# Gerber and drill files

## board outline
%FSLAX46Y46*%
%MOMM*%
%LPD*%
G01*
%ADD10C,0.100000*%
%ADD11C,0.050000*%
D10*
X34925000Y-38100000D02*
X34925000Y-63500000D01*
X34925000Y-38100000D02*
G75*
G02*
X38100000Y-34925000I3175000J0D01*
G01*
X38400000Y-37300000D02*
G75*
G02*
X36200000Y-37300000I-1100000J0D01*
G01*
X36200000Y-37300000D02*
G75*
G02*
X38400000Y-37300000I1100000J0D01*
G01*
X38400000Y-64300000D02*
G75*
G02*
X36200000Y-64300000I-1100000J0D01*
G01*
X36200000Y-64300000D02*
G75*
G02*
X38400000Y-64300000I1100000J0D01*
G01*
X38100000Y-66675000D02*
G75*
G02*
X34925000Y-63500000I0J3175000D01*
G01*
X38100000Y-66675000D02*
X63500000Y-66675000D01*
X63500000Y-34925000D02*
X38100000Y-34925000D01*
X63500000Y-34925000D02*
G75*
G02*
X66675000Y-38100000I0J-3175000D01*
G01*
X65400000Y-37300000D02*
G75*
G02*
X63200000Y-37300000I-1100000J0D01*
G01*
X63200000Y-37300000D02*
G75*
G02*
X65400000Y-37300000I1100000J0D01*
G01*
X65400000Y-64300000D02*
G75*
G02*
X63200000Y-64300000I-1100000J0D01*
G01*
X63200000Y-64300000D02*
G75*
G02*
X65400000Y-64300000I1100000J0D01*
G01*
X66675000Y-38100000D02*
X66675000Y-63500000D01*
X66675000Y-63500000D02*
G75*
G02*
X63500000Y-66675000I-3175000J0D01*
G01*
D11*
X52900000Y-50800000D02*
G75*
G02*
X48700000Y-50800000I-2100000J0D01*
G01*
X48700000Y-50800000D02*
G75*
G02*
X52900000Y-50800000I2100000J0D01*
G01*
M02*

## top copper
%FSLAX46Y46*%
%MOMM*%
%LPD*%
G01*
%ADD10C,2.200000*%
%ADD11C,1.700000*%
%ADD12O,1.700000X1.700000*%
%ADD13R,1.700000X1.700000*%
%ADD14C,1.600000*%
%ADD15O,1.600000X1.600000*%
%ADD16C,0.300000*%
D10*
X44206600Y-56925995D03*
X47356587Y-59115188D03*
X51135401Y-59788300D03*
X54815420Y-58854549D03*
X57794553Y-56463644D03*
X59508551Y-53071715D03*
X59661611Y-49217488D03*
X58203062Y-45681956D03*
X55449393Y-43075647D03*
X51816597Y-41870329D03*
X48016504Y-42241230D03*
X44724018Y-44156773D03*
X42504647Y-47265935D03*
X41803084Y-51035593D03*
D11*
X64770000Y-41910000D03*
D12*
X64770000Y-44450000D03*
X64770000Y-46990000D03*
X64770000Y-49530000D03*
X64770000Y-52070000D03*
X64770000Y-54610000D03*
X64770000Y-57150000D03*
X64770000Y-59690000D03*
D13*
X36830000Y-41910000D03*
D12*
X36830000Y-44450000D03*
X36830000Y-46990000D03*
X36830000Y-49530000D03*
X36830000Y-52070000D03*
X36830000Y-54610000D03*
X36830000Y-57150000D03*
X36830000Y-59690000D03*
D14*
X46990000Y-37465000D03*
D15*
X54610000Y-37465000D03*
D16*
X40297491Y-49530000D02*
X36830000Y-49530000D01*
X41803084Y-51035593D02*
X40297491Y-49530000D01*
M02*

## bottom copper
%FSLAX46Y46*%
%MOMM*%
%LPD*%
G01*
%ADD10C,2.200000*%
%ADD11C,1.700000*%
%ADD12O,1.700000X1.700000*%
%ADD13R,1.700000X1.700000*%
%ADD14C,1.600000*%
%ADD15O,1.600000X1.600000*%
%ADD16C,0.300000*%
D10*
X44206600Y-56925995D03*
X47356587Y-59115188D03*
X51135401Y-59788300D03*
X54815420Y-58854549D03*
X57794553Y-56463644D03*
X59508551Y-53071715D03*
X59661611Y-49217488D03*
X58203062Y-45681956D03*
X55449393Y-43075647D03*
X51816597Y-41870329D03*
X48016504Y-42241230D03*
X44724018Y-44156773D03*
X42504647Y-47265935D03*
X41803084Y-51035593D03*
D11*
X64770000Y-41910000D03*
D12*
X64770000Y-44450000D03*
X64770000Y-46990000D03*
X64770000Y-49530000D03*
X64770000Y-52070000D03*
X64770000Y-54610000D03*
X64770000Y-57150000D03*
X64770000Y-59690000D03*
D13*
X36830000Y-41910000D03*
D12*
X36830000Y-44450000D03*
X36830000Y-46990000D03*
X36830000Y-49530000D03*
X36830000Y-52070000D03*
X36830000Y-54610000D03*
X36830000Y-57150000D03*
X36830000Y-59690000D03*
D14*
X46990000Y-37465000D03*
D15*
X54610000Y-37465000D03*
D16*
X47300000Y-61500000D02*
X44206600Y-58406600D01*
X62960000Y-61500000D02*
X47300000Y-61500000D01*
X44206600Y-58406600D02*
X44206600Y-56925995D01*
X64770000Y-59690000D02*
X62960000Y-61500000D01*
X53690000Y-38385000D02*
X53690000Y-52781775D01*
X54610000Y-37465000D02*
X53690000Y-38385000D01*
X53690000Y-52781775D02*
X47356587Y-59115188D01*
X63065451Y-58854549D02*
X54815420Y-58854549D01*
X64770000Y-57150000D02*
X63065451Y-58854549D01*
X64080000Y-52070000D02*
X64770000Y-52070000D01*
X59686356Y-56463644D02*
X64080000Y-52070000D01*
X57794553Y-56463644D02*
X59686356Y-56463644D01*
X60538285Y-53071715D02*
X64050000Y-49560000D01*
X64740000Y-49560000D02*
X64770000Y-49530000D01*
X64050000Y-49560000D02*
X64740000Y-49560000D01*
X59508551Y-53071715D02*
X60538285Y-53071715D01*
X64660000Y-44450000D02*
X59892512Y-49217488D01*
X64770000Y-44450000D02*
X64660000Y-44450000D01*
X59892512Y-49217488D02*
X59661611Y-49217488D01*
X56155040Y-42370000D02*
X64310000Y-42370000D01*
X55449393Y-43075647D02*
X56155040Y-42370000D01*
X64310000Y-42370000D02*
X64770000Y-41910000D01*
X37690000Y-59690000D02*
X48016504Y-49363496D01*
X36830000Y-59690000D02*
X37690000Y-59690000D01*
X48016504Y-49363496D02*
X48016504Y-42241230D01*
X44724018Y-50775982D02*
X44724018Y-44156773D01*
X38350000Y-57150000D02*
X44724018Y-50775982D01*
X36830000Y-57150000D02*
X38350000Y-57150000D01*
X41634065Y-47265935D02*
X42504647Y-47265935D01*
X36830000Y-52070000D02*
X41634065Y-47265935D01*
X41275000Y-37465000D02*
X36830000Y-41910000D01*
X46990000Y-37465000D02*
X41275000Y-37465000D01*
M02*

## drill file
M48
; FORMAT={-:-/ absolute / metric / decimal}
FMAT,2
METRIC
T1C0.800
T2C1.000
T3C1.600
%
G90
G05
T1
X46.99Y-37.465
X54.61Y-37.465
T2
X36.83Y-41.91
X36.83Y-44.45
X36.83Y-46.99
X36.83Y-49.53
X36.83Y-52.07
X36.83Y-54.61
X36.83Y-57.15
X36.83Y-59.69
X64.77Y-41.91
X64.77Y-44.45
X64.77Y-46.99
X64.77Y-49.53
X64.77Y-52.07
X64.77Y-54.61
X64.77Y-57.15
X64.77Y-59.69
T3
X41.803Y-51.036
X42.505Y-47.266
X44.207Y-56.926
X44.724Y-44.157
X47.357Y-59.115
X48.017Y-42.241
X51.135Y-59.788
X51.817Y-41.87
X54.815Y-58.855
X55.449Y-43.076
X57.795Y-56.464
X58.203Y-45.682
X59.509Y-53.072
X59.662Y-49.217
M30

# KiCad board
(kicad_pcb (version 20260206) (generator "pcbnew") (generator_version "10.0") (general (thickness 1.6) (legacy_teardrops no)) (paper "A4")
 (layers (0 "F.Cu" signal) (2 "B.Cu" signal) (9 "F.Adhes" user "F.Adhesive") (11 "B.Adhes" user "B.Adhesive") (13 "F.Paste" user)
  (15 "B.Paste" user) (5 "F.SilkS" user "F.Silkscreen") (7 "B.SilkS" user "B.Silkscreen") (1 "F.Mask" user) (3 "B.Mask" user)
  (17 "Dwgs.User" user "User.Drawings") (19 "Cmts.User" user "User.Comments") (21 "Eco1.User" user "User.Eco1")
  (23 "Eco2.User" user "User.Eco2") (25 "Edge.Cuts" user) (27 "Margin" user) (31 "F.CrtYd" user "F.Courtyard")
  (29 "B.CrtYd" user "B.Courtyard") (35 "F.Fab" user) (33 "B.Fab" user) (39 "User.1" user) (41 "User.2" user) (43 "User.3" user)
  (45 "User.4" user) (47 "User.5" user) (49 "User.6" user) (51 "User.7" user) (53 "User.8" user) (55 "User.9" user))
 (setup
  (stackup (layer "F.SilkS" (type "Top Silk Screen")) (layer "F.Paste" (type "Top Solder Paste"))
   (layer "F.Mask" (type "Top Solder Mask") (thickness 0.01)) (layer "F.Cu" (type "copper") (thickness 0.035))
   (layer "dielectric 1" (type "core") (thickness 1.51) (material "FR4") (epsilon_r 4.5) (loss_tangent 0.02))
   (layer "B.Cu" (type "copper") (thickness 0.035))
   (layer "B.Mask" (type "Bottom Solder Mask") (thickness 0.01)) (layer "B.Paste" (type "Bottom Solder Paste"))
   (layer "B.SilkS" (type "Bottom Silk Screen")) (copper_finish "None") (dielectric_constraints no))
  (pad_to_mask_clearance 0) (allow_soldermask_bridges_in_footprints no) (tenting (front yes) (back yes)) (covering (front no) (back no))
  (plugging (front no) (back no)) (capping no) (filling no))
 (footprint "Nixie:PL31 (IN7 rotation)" (layer "F.Cu") (at 50.8 50.8 -90)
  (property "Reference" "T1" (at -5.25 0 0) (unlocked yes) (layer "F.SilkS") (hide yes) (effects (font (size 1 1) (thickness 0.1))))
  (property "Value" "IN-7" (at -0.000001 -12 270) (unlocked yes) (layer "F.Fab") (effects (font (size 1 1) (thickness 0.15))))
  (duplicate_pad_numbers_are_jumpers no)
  (fp_circle (center 0 0) (end 2.1 0) (stroke (width 0.05) (type default)) (fill no) (layer "Edge.Cuts"))
  (pad "1" thru_hole circle (at 6.125995 6.5934 91.5) (size 2.2 2.2) (drill 1.6) (layers "*.Cu" "*.Mask") (remove_unused_layers no)
   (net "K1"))
  (pad "2" thru_hole circle (at 8.315188 3.443413 91.5) (size 2.2 2.2) (drill 1.6) (layers "*.Cu" "*.Mask") (remove_unused_layers no)
   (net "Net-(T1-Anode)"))
  (pad "3" thru_hole circle (at 8.9883 -0.335401 91.5) (size 2.2 2.2) (drill 1.6) (layers "*.Cu" "*.Mask") (remove_unused_layers no)
   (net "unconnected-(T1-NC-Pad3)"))
  (pad "4" thru_hole circle (at 8.054549 -4.01542 91.5) (size 2.2 2.2) (drill 1.6) (layers "*.Cu" "*.Mask") (remove_unused_layers no)
   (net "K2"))
  (pad "5" thru_hole circle (at 5.663644 -6.994553 91.5) (size 2.2 2.2) (drill 1.6) (layers "*.Cu" "*.Mask") (remove_unused_layers no)
   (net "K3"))
  (pad "6" thru_hole circle (at 2.271715 -8.708551 91.5) (size 2.2 2.2) (drill 1.6) (layers "*.Cu" "*.Mask") (remove_unused_layers no)
   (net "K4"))
  (pad "7" thru_hole circle (at -1.582512 -8.861611 91.5) (size 2.2 2.2) (drill 1.6) (layers "*.Cu" "*.Mask") (remove_unused_layers no)
   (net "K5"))
  (pad "8" thru_hole circle (at -5.118044 -7.403062 91.5) (size 2.2 2.2) (drill 1.6) (layers "*.Cu" "*.Mask") (remove_unused_layers no)
   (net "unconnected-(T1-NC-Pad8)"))
  (pad "9" thru_hole circle (at -7.724353 -4.649393 91.5) (size 2.2 2.2) (drill 1.6) (layers "*.Cu" "*.Mask") (remove_unused_layers no)
   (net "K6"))
  (pad "10" thru_hole circle (at -8.929671 -1.016597 91.5) (size 2.2 2.2) (drill 1.6) (layers "*.Cu" "*.Mask") (remove_unused_layers no)
   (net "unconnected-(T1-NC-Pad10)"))
  (pad "11" thru_hole circle (at -8.55877 2.783496 91.5) (size 2.2 2.2) (drill 1.6) (layers "*.Cu" "*.Mask") (remove_unused_layers no)
   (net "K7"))
  (pad "12" thru_hole circle (at -6.643227 6.075982 91.5) (size 2.2 2.2) (drill 1.6) (layers "*.Cu" "*.Mask") (remove_unused_layers no)
   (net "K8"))
  (pad "13" thru_hole circle (at -3.534065 8.295353 91.5) (size 2.2 2.2) (drill 1.6) (layers "*.Cu" "*.Mask") (remove_unused_layers no)
   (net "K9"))
  (pad "14" thru_hole circle (at 0.235593 8.996916 91.5) (size 2.2 2.2) (drill 1.6) (layers "*.Cu" "*.Mask") (remove_unused_layers no)
   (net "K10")))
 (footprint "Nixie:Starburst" (layer "F.Cu") (at 43 63.25)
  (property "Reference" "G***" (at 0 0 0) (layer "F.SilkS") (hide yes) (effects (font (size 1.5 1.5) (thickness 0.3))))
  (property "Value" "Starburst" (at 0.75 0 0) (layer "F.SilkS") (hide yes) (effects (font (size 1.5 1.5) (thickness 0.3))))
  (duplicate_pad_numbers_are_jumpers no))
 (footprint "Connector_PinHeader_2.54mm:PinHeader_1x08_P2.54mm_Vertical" (layer "B.Cu") (at 64.77 41.91 180)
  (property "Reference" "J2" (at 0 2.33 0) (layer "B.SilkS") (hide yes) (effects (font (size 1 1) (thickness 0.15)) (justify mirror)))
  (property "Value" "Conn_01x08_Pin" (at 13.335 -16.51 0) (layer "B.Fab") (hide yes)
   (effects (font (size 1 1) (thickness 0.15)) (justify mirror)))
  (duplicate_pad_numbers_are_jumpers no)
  (pad "1" thru_hole circle (at 0 0 180) (size 1.7 1.7) (drill 1) (layers "*.Cu" "*.Mask") (remove_unused_layers no) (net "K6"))
  (pad "2" thru_hole oval (at 0 -2.54 180) (size 1.7 1.7) (drill 1) (layers "*.Cu" "*.Mask") (remove_unused_layers no) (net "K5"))
  (pad "3" thru_hole oval (at 0 -5.08 180) (size 1.7 1.7) (drill 1) (layers "*.Cu" "*.Mask") (remove_unused_layers no)
   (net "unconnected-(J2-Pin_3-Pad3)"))
  (pad "4" thru_hole oval (at 0 -7.62 180) (size 1.7 1.7) (drill 1) (layers "*.Cu" "*.Mask") (remove_unused_layers no) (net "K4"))
  (pad "5" thru_hole oval (at 0 -10.16 180) (size 1.7 1.7) (drill 1) (layers "*.Cu" "*.Mask") (remove_unused_layers no) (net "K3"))
  (pad "6" thru_hole oval (at 0 -12.7 180) (size 1.7 1.7) (drill 1) (layers "*.Cu" "*.Mask") (remove_unused_layers no)
   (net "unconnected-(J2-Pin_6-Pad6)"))
  (pad "7" thru_hole oval (at 0 -15.24 180) (size 1.7 1.7) (drill 1) (layers "*.Cu" "*.Mask") (remove_unused_layers no) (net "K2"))
  (pad "8" thru_hole oval (at 0 -17.78 180) (size 1.7 1.7) (drill 1) (layers "*.Cu" "*.Mask") (remove_unused_layers no) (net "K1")))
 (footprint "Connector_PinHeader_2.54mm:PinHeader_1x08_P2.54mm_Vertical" (layer "B.Cu") (at 36.83 41.91 180)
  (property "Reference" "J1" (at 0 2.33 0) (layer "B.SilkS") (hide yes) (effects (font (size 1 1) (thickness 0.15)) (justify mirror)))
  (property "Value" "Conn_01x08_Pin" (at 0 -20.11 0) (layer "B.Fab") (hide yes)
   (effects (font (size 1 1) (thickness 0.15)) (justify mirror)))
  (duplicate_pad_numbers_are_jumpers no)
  (pad "1" thru_hole rect (at 0 0 180) (size 1.7 1.7) (drill 1) (layers "*.Cu" "*.Mask") (remove_unused_layers no) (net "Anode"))
  (pad "2" thru_hole oval (at 0 -2.54 180) (size 1.7 1.7) (drill 1) (layers "*.Cu" "*.Mask") (remove_unused_layers no)
   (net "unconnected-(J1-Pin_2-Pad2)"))
  (pad "3" thru_hole oval (at 0 -5.08 180) (size 1.7 1.7) (drill 1) (layers "*.Cu" "*.Mask") (remove_unused_layers no)
   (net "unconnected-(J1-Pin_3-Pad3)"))
  (pad "4" thru_hole oval (at 0 -7.62 180) (size 1.7 1.7) (drill 1) (layers "*.Cu" "*.Mask") (remove_unused_layers no) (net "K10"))
  (pad "5" thru_hole oval (at 0 -10.16 180) (size 1.7 1.7) (drill 1) (layers "*.Cu" "*.Mask") (remove_unused_layers no) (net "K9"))
  (pad "6" thru_hole oval (at 0 -12.7 180) (size 1.7 1.7) (drill 1) (layers "*.Cu" "*.Mask") (remove_unused_layers no)
   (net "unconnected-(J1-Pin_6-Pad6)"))
  (pad "7" thru_hole oval (at 0 -15.24 180) (size 1.7 1.7) (drill 1) (layers "*.Cu" "*.Mask") (remove_unused_layers no) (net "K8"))
  (pad "8" thru_hole oval (at 0 -17.78 180) (size 1.7 1.7) (drill 1) (layers "*.Cu" "*.Mask") (remove_unused_layers no) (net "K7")))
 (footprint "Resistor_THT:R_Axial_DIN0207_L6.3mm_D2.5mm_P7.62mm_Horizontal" (layer "B.Cu") (at 46.99 37.465)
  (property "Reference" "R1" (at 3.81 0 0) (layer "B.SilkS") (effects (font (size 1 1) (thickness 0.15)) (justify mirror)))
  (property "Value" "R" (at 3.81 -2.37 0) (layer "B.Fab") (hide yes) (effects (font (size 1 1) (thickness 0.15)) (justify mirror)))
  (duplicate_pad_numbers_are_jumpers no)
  (pad "1" thru_hole circle (at 0 0) (size 1.6 1.6) (drill 0.8) (layers "*.Cu" "*.Mask") (remove_unused_layers no) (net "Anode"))
  (pad "2" thru_hole oval (at 7.62 0) (size 1.6 1.6) (drill 0.8) (layers "*.Cu" "*.Mask") (remove_unused_layers no) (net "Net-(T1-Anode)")))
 (gr_line (start 34.925 38.1) (end 34.925 63.5) (stroke (width 0.1) (type default)) (layer "Edge.Cuts"))
 (gr_arc (start 34.925 38.1) (mid 35.854936 35.854936) (end 38.1 34.925) (stroke (width 0.1) (type default)) (layer "Edge.Cuts"))
 (gr_circle (center 37.3 37.3) (end 38.4 37.3) (stroke (width 0.1) (type default)) (fill no) (layer "Edge.Cuts"))
 (gr_circle (center 37.3 64.3) (end 38.4 64.3) (stroke (width 0.1) (type default)) (fill no) (layer "Edge.Cuts"))
 (gr_arc (start 38.1 66.675) (mid 35.854936 65.745064) (end 34.925 63.5) (stroke (width 0.1) (type default)) (layer "Edge.Cuts"))
 (gr_line (start 38.1 66.675) (end 63.5 66.675) (stroke (width 0.1) (type default)) (layer "Edge.Cuts"))
 (gr_line (start 63.5 34.925) (end 38.1 34.925) (stroke (width 0.1) (type default)) (layer "Edge.Cuts"))
 (gr_arc (start 63.5 34.925) (mid 65.745064 35.854936) (end 66.675 38.1) (stroke (width 0.1) (type default)) (layer "Edge.Cuts"))
 (gr_circle (center 64.3 37.3) (end 65.4 37.3) (stroke (width 0.1) (type default)) (fill no) (layer "Edge.Cuts"))
 (gr_circle (center 64.3 64.3) (end 65.4 64.3) (stroke (width 0.1) (type default)) (fill no) (layer "Edge.Cuts"))
 (gr_line (start 66.675 38.1) (end 66.675 63.5) (stroke (width 0.1) (type default)) (layer "Edge.Cuts"))
 (gr_arc (start 66.675 63.5) (mid 65.745064 65.745064) (end 63.5 66.675) (stroke (width 0.1) (type default)) (layer "Edge.Cuts"))
 (segment (start 47.3 61.5) (end 44.2066 58.4066) (width 0.3) (layer "B.Cu") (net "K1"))
 (segment (start 62.96 61.5) (end 47.3 61.5) (width 0.3) (layer "B.Cu") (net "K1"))
 (segment (start 44.2066 58.4066) (end 44.2066 56.925995) (width 0.3) (layer "B.Cu") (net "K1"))
 (segment (start 64.77 59.69) (end 62.96 61.5) (width 0.3) (layer "B.Cu") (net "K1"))
 (segment (start 53.69 38.385) (end 53.69 52.781775) (width 0.3) (layer "B.Cu") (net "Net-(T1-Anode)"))
 (segment (start 54.61 37.465) (end 53.69 38.385) (width 0.3) (layer "B.Cu") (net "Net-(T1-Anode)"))
 (segment (start 53.69 52.781775) (end 47.356587 59.115188) (width 0.3) (layer "B.Cu") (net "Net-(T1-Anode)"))
 (segment (start 63.065451 58.854549) (end 54.81542 58.854549) (width 0.3) (layer "B.Cu") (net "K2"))
 (segment (start 64.77 57.15) (end 63.065451 58.854549) (width 0.3) (layer "B.Cu") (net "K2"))
 (segment (start 64.08 52.07) (end 64.77 52.07) (width 0.3) (layer "B.Cu") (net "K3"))
 (segment (start 59.686356 56.463644) (end 64.08 52.07) (width 0.3) (layer "B.Cu") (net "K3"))
 (segment (start 57.794553 56.463644) (end 59.686356 56.463644) (width 0.3) (layer "B.Cu") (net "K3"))
 (segment (start 60.538285 53.071715) (end 64.05 49.56) (width 0.3) (layer "B.Cu") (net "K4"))
 (segment (start 64.74 49.56) (end 64.77 49.53) (width 0.3) (layer "B.Cu") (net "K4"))
 (segment (start 64.05 49.56) (end 64.74 49.56) (width 0.3) (layer "B.Cu") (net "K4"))
 (segment (start 59.508551 53.071715) (end 60.538285 53.071715) (width 0.3) (layer "B.Cu") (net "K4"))
 (segment (start 64.66 44.45) (end 59.892512 49.217488) (width 0.3) (layer "B.Cu") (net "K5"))
 (segment (start 64.77 44.45) (end 64.66 44.45) (width 0.3) (layer "B.Cu") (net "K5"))
 (segment (start 59.892512 49.217488) (end 59.661611 49.217488) (width 0.3) (layer "B.Cu") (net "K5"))
 (segment (start 56.15504 42.37) (end 64.31 42.37) (width 0.3) (layer "B.Cu") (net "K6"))
 (segment (start 55.449393 43.075647) (end 56.15504 42.37) (width 0.3) (layer "B.Cu") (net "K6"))
 (segment (start 64.31 42.37) (end 64.77 41.91) (width 0.3) (layer "B.Cu") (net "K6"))
 (segment (start 37.69 59.69) (end 48.016504 49.363496) (width 0.3) (layer "B.Cu") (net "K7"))
 (segment (start 36.83 59.69) (end 37.69 59.69) (width 0.3) (layer "B.Cu") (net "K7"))
 (segment (start 48.016504 49.363496) (end 48.016504 42.24123) (width 0.3) (layer "B.Cu") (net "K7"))
 (segment (start 44.724018 50.775982) (end 44.724018 44.156773) (width 0.3) (layer "B.Cu") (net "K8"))
 (segment (start 38.35 57.15) (end 44.724018 50.775982) (width 0.3) (layer "B.Cu") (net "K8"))
 (segment (start 36.83 57.15) (end 38.35 57.15) (width 0.3) (layer "B.Cu") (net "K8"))
 (segment (start 41.634065 47.265935) (end 42.504647 47.265935) (width 0.3) (layer "B.Cu") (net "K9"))
 (segment (start 36.83 52.07) (end 41.634065 47.265935) (width 0.3) (layer "B.Cu") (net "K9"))
 (segment (start 40.297491 49.53) (end 36.83 49.53) (width 0.3) (layer "F.Cu") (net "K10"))
 (segment (start 41.803084 51.035593) (end 40.297491 49.53) (width 0.3) (layer "F.Cu") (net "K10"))
 (segment (start 41.275 37.465) (end 36.83 41.91) (width 0.3) (layer "B.Cu") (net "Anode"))
 (segment (start 46.99 37.465) (end 41.275 37.465) (width 0.3) (layer "B.Cu") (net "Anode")))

